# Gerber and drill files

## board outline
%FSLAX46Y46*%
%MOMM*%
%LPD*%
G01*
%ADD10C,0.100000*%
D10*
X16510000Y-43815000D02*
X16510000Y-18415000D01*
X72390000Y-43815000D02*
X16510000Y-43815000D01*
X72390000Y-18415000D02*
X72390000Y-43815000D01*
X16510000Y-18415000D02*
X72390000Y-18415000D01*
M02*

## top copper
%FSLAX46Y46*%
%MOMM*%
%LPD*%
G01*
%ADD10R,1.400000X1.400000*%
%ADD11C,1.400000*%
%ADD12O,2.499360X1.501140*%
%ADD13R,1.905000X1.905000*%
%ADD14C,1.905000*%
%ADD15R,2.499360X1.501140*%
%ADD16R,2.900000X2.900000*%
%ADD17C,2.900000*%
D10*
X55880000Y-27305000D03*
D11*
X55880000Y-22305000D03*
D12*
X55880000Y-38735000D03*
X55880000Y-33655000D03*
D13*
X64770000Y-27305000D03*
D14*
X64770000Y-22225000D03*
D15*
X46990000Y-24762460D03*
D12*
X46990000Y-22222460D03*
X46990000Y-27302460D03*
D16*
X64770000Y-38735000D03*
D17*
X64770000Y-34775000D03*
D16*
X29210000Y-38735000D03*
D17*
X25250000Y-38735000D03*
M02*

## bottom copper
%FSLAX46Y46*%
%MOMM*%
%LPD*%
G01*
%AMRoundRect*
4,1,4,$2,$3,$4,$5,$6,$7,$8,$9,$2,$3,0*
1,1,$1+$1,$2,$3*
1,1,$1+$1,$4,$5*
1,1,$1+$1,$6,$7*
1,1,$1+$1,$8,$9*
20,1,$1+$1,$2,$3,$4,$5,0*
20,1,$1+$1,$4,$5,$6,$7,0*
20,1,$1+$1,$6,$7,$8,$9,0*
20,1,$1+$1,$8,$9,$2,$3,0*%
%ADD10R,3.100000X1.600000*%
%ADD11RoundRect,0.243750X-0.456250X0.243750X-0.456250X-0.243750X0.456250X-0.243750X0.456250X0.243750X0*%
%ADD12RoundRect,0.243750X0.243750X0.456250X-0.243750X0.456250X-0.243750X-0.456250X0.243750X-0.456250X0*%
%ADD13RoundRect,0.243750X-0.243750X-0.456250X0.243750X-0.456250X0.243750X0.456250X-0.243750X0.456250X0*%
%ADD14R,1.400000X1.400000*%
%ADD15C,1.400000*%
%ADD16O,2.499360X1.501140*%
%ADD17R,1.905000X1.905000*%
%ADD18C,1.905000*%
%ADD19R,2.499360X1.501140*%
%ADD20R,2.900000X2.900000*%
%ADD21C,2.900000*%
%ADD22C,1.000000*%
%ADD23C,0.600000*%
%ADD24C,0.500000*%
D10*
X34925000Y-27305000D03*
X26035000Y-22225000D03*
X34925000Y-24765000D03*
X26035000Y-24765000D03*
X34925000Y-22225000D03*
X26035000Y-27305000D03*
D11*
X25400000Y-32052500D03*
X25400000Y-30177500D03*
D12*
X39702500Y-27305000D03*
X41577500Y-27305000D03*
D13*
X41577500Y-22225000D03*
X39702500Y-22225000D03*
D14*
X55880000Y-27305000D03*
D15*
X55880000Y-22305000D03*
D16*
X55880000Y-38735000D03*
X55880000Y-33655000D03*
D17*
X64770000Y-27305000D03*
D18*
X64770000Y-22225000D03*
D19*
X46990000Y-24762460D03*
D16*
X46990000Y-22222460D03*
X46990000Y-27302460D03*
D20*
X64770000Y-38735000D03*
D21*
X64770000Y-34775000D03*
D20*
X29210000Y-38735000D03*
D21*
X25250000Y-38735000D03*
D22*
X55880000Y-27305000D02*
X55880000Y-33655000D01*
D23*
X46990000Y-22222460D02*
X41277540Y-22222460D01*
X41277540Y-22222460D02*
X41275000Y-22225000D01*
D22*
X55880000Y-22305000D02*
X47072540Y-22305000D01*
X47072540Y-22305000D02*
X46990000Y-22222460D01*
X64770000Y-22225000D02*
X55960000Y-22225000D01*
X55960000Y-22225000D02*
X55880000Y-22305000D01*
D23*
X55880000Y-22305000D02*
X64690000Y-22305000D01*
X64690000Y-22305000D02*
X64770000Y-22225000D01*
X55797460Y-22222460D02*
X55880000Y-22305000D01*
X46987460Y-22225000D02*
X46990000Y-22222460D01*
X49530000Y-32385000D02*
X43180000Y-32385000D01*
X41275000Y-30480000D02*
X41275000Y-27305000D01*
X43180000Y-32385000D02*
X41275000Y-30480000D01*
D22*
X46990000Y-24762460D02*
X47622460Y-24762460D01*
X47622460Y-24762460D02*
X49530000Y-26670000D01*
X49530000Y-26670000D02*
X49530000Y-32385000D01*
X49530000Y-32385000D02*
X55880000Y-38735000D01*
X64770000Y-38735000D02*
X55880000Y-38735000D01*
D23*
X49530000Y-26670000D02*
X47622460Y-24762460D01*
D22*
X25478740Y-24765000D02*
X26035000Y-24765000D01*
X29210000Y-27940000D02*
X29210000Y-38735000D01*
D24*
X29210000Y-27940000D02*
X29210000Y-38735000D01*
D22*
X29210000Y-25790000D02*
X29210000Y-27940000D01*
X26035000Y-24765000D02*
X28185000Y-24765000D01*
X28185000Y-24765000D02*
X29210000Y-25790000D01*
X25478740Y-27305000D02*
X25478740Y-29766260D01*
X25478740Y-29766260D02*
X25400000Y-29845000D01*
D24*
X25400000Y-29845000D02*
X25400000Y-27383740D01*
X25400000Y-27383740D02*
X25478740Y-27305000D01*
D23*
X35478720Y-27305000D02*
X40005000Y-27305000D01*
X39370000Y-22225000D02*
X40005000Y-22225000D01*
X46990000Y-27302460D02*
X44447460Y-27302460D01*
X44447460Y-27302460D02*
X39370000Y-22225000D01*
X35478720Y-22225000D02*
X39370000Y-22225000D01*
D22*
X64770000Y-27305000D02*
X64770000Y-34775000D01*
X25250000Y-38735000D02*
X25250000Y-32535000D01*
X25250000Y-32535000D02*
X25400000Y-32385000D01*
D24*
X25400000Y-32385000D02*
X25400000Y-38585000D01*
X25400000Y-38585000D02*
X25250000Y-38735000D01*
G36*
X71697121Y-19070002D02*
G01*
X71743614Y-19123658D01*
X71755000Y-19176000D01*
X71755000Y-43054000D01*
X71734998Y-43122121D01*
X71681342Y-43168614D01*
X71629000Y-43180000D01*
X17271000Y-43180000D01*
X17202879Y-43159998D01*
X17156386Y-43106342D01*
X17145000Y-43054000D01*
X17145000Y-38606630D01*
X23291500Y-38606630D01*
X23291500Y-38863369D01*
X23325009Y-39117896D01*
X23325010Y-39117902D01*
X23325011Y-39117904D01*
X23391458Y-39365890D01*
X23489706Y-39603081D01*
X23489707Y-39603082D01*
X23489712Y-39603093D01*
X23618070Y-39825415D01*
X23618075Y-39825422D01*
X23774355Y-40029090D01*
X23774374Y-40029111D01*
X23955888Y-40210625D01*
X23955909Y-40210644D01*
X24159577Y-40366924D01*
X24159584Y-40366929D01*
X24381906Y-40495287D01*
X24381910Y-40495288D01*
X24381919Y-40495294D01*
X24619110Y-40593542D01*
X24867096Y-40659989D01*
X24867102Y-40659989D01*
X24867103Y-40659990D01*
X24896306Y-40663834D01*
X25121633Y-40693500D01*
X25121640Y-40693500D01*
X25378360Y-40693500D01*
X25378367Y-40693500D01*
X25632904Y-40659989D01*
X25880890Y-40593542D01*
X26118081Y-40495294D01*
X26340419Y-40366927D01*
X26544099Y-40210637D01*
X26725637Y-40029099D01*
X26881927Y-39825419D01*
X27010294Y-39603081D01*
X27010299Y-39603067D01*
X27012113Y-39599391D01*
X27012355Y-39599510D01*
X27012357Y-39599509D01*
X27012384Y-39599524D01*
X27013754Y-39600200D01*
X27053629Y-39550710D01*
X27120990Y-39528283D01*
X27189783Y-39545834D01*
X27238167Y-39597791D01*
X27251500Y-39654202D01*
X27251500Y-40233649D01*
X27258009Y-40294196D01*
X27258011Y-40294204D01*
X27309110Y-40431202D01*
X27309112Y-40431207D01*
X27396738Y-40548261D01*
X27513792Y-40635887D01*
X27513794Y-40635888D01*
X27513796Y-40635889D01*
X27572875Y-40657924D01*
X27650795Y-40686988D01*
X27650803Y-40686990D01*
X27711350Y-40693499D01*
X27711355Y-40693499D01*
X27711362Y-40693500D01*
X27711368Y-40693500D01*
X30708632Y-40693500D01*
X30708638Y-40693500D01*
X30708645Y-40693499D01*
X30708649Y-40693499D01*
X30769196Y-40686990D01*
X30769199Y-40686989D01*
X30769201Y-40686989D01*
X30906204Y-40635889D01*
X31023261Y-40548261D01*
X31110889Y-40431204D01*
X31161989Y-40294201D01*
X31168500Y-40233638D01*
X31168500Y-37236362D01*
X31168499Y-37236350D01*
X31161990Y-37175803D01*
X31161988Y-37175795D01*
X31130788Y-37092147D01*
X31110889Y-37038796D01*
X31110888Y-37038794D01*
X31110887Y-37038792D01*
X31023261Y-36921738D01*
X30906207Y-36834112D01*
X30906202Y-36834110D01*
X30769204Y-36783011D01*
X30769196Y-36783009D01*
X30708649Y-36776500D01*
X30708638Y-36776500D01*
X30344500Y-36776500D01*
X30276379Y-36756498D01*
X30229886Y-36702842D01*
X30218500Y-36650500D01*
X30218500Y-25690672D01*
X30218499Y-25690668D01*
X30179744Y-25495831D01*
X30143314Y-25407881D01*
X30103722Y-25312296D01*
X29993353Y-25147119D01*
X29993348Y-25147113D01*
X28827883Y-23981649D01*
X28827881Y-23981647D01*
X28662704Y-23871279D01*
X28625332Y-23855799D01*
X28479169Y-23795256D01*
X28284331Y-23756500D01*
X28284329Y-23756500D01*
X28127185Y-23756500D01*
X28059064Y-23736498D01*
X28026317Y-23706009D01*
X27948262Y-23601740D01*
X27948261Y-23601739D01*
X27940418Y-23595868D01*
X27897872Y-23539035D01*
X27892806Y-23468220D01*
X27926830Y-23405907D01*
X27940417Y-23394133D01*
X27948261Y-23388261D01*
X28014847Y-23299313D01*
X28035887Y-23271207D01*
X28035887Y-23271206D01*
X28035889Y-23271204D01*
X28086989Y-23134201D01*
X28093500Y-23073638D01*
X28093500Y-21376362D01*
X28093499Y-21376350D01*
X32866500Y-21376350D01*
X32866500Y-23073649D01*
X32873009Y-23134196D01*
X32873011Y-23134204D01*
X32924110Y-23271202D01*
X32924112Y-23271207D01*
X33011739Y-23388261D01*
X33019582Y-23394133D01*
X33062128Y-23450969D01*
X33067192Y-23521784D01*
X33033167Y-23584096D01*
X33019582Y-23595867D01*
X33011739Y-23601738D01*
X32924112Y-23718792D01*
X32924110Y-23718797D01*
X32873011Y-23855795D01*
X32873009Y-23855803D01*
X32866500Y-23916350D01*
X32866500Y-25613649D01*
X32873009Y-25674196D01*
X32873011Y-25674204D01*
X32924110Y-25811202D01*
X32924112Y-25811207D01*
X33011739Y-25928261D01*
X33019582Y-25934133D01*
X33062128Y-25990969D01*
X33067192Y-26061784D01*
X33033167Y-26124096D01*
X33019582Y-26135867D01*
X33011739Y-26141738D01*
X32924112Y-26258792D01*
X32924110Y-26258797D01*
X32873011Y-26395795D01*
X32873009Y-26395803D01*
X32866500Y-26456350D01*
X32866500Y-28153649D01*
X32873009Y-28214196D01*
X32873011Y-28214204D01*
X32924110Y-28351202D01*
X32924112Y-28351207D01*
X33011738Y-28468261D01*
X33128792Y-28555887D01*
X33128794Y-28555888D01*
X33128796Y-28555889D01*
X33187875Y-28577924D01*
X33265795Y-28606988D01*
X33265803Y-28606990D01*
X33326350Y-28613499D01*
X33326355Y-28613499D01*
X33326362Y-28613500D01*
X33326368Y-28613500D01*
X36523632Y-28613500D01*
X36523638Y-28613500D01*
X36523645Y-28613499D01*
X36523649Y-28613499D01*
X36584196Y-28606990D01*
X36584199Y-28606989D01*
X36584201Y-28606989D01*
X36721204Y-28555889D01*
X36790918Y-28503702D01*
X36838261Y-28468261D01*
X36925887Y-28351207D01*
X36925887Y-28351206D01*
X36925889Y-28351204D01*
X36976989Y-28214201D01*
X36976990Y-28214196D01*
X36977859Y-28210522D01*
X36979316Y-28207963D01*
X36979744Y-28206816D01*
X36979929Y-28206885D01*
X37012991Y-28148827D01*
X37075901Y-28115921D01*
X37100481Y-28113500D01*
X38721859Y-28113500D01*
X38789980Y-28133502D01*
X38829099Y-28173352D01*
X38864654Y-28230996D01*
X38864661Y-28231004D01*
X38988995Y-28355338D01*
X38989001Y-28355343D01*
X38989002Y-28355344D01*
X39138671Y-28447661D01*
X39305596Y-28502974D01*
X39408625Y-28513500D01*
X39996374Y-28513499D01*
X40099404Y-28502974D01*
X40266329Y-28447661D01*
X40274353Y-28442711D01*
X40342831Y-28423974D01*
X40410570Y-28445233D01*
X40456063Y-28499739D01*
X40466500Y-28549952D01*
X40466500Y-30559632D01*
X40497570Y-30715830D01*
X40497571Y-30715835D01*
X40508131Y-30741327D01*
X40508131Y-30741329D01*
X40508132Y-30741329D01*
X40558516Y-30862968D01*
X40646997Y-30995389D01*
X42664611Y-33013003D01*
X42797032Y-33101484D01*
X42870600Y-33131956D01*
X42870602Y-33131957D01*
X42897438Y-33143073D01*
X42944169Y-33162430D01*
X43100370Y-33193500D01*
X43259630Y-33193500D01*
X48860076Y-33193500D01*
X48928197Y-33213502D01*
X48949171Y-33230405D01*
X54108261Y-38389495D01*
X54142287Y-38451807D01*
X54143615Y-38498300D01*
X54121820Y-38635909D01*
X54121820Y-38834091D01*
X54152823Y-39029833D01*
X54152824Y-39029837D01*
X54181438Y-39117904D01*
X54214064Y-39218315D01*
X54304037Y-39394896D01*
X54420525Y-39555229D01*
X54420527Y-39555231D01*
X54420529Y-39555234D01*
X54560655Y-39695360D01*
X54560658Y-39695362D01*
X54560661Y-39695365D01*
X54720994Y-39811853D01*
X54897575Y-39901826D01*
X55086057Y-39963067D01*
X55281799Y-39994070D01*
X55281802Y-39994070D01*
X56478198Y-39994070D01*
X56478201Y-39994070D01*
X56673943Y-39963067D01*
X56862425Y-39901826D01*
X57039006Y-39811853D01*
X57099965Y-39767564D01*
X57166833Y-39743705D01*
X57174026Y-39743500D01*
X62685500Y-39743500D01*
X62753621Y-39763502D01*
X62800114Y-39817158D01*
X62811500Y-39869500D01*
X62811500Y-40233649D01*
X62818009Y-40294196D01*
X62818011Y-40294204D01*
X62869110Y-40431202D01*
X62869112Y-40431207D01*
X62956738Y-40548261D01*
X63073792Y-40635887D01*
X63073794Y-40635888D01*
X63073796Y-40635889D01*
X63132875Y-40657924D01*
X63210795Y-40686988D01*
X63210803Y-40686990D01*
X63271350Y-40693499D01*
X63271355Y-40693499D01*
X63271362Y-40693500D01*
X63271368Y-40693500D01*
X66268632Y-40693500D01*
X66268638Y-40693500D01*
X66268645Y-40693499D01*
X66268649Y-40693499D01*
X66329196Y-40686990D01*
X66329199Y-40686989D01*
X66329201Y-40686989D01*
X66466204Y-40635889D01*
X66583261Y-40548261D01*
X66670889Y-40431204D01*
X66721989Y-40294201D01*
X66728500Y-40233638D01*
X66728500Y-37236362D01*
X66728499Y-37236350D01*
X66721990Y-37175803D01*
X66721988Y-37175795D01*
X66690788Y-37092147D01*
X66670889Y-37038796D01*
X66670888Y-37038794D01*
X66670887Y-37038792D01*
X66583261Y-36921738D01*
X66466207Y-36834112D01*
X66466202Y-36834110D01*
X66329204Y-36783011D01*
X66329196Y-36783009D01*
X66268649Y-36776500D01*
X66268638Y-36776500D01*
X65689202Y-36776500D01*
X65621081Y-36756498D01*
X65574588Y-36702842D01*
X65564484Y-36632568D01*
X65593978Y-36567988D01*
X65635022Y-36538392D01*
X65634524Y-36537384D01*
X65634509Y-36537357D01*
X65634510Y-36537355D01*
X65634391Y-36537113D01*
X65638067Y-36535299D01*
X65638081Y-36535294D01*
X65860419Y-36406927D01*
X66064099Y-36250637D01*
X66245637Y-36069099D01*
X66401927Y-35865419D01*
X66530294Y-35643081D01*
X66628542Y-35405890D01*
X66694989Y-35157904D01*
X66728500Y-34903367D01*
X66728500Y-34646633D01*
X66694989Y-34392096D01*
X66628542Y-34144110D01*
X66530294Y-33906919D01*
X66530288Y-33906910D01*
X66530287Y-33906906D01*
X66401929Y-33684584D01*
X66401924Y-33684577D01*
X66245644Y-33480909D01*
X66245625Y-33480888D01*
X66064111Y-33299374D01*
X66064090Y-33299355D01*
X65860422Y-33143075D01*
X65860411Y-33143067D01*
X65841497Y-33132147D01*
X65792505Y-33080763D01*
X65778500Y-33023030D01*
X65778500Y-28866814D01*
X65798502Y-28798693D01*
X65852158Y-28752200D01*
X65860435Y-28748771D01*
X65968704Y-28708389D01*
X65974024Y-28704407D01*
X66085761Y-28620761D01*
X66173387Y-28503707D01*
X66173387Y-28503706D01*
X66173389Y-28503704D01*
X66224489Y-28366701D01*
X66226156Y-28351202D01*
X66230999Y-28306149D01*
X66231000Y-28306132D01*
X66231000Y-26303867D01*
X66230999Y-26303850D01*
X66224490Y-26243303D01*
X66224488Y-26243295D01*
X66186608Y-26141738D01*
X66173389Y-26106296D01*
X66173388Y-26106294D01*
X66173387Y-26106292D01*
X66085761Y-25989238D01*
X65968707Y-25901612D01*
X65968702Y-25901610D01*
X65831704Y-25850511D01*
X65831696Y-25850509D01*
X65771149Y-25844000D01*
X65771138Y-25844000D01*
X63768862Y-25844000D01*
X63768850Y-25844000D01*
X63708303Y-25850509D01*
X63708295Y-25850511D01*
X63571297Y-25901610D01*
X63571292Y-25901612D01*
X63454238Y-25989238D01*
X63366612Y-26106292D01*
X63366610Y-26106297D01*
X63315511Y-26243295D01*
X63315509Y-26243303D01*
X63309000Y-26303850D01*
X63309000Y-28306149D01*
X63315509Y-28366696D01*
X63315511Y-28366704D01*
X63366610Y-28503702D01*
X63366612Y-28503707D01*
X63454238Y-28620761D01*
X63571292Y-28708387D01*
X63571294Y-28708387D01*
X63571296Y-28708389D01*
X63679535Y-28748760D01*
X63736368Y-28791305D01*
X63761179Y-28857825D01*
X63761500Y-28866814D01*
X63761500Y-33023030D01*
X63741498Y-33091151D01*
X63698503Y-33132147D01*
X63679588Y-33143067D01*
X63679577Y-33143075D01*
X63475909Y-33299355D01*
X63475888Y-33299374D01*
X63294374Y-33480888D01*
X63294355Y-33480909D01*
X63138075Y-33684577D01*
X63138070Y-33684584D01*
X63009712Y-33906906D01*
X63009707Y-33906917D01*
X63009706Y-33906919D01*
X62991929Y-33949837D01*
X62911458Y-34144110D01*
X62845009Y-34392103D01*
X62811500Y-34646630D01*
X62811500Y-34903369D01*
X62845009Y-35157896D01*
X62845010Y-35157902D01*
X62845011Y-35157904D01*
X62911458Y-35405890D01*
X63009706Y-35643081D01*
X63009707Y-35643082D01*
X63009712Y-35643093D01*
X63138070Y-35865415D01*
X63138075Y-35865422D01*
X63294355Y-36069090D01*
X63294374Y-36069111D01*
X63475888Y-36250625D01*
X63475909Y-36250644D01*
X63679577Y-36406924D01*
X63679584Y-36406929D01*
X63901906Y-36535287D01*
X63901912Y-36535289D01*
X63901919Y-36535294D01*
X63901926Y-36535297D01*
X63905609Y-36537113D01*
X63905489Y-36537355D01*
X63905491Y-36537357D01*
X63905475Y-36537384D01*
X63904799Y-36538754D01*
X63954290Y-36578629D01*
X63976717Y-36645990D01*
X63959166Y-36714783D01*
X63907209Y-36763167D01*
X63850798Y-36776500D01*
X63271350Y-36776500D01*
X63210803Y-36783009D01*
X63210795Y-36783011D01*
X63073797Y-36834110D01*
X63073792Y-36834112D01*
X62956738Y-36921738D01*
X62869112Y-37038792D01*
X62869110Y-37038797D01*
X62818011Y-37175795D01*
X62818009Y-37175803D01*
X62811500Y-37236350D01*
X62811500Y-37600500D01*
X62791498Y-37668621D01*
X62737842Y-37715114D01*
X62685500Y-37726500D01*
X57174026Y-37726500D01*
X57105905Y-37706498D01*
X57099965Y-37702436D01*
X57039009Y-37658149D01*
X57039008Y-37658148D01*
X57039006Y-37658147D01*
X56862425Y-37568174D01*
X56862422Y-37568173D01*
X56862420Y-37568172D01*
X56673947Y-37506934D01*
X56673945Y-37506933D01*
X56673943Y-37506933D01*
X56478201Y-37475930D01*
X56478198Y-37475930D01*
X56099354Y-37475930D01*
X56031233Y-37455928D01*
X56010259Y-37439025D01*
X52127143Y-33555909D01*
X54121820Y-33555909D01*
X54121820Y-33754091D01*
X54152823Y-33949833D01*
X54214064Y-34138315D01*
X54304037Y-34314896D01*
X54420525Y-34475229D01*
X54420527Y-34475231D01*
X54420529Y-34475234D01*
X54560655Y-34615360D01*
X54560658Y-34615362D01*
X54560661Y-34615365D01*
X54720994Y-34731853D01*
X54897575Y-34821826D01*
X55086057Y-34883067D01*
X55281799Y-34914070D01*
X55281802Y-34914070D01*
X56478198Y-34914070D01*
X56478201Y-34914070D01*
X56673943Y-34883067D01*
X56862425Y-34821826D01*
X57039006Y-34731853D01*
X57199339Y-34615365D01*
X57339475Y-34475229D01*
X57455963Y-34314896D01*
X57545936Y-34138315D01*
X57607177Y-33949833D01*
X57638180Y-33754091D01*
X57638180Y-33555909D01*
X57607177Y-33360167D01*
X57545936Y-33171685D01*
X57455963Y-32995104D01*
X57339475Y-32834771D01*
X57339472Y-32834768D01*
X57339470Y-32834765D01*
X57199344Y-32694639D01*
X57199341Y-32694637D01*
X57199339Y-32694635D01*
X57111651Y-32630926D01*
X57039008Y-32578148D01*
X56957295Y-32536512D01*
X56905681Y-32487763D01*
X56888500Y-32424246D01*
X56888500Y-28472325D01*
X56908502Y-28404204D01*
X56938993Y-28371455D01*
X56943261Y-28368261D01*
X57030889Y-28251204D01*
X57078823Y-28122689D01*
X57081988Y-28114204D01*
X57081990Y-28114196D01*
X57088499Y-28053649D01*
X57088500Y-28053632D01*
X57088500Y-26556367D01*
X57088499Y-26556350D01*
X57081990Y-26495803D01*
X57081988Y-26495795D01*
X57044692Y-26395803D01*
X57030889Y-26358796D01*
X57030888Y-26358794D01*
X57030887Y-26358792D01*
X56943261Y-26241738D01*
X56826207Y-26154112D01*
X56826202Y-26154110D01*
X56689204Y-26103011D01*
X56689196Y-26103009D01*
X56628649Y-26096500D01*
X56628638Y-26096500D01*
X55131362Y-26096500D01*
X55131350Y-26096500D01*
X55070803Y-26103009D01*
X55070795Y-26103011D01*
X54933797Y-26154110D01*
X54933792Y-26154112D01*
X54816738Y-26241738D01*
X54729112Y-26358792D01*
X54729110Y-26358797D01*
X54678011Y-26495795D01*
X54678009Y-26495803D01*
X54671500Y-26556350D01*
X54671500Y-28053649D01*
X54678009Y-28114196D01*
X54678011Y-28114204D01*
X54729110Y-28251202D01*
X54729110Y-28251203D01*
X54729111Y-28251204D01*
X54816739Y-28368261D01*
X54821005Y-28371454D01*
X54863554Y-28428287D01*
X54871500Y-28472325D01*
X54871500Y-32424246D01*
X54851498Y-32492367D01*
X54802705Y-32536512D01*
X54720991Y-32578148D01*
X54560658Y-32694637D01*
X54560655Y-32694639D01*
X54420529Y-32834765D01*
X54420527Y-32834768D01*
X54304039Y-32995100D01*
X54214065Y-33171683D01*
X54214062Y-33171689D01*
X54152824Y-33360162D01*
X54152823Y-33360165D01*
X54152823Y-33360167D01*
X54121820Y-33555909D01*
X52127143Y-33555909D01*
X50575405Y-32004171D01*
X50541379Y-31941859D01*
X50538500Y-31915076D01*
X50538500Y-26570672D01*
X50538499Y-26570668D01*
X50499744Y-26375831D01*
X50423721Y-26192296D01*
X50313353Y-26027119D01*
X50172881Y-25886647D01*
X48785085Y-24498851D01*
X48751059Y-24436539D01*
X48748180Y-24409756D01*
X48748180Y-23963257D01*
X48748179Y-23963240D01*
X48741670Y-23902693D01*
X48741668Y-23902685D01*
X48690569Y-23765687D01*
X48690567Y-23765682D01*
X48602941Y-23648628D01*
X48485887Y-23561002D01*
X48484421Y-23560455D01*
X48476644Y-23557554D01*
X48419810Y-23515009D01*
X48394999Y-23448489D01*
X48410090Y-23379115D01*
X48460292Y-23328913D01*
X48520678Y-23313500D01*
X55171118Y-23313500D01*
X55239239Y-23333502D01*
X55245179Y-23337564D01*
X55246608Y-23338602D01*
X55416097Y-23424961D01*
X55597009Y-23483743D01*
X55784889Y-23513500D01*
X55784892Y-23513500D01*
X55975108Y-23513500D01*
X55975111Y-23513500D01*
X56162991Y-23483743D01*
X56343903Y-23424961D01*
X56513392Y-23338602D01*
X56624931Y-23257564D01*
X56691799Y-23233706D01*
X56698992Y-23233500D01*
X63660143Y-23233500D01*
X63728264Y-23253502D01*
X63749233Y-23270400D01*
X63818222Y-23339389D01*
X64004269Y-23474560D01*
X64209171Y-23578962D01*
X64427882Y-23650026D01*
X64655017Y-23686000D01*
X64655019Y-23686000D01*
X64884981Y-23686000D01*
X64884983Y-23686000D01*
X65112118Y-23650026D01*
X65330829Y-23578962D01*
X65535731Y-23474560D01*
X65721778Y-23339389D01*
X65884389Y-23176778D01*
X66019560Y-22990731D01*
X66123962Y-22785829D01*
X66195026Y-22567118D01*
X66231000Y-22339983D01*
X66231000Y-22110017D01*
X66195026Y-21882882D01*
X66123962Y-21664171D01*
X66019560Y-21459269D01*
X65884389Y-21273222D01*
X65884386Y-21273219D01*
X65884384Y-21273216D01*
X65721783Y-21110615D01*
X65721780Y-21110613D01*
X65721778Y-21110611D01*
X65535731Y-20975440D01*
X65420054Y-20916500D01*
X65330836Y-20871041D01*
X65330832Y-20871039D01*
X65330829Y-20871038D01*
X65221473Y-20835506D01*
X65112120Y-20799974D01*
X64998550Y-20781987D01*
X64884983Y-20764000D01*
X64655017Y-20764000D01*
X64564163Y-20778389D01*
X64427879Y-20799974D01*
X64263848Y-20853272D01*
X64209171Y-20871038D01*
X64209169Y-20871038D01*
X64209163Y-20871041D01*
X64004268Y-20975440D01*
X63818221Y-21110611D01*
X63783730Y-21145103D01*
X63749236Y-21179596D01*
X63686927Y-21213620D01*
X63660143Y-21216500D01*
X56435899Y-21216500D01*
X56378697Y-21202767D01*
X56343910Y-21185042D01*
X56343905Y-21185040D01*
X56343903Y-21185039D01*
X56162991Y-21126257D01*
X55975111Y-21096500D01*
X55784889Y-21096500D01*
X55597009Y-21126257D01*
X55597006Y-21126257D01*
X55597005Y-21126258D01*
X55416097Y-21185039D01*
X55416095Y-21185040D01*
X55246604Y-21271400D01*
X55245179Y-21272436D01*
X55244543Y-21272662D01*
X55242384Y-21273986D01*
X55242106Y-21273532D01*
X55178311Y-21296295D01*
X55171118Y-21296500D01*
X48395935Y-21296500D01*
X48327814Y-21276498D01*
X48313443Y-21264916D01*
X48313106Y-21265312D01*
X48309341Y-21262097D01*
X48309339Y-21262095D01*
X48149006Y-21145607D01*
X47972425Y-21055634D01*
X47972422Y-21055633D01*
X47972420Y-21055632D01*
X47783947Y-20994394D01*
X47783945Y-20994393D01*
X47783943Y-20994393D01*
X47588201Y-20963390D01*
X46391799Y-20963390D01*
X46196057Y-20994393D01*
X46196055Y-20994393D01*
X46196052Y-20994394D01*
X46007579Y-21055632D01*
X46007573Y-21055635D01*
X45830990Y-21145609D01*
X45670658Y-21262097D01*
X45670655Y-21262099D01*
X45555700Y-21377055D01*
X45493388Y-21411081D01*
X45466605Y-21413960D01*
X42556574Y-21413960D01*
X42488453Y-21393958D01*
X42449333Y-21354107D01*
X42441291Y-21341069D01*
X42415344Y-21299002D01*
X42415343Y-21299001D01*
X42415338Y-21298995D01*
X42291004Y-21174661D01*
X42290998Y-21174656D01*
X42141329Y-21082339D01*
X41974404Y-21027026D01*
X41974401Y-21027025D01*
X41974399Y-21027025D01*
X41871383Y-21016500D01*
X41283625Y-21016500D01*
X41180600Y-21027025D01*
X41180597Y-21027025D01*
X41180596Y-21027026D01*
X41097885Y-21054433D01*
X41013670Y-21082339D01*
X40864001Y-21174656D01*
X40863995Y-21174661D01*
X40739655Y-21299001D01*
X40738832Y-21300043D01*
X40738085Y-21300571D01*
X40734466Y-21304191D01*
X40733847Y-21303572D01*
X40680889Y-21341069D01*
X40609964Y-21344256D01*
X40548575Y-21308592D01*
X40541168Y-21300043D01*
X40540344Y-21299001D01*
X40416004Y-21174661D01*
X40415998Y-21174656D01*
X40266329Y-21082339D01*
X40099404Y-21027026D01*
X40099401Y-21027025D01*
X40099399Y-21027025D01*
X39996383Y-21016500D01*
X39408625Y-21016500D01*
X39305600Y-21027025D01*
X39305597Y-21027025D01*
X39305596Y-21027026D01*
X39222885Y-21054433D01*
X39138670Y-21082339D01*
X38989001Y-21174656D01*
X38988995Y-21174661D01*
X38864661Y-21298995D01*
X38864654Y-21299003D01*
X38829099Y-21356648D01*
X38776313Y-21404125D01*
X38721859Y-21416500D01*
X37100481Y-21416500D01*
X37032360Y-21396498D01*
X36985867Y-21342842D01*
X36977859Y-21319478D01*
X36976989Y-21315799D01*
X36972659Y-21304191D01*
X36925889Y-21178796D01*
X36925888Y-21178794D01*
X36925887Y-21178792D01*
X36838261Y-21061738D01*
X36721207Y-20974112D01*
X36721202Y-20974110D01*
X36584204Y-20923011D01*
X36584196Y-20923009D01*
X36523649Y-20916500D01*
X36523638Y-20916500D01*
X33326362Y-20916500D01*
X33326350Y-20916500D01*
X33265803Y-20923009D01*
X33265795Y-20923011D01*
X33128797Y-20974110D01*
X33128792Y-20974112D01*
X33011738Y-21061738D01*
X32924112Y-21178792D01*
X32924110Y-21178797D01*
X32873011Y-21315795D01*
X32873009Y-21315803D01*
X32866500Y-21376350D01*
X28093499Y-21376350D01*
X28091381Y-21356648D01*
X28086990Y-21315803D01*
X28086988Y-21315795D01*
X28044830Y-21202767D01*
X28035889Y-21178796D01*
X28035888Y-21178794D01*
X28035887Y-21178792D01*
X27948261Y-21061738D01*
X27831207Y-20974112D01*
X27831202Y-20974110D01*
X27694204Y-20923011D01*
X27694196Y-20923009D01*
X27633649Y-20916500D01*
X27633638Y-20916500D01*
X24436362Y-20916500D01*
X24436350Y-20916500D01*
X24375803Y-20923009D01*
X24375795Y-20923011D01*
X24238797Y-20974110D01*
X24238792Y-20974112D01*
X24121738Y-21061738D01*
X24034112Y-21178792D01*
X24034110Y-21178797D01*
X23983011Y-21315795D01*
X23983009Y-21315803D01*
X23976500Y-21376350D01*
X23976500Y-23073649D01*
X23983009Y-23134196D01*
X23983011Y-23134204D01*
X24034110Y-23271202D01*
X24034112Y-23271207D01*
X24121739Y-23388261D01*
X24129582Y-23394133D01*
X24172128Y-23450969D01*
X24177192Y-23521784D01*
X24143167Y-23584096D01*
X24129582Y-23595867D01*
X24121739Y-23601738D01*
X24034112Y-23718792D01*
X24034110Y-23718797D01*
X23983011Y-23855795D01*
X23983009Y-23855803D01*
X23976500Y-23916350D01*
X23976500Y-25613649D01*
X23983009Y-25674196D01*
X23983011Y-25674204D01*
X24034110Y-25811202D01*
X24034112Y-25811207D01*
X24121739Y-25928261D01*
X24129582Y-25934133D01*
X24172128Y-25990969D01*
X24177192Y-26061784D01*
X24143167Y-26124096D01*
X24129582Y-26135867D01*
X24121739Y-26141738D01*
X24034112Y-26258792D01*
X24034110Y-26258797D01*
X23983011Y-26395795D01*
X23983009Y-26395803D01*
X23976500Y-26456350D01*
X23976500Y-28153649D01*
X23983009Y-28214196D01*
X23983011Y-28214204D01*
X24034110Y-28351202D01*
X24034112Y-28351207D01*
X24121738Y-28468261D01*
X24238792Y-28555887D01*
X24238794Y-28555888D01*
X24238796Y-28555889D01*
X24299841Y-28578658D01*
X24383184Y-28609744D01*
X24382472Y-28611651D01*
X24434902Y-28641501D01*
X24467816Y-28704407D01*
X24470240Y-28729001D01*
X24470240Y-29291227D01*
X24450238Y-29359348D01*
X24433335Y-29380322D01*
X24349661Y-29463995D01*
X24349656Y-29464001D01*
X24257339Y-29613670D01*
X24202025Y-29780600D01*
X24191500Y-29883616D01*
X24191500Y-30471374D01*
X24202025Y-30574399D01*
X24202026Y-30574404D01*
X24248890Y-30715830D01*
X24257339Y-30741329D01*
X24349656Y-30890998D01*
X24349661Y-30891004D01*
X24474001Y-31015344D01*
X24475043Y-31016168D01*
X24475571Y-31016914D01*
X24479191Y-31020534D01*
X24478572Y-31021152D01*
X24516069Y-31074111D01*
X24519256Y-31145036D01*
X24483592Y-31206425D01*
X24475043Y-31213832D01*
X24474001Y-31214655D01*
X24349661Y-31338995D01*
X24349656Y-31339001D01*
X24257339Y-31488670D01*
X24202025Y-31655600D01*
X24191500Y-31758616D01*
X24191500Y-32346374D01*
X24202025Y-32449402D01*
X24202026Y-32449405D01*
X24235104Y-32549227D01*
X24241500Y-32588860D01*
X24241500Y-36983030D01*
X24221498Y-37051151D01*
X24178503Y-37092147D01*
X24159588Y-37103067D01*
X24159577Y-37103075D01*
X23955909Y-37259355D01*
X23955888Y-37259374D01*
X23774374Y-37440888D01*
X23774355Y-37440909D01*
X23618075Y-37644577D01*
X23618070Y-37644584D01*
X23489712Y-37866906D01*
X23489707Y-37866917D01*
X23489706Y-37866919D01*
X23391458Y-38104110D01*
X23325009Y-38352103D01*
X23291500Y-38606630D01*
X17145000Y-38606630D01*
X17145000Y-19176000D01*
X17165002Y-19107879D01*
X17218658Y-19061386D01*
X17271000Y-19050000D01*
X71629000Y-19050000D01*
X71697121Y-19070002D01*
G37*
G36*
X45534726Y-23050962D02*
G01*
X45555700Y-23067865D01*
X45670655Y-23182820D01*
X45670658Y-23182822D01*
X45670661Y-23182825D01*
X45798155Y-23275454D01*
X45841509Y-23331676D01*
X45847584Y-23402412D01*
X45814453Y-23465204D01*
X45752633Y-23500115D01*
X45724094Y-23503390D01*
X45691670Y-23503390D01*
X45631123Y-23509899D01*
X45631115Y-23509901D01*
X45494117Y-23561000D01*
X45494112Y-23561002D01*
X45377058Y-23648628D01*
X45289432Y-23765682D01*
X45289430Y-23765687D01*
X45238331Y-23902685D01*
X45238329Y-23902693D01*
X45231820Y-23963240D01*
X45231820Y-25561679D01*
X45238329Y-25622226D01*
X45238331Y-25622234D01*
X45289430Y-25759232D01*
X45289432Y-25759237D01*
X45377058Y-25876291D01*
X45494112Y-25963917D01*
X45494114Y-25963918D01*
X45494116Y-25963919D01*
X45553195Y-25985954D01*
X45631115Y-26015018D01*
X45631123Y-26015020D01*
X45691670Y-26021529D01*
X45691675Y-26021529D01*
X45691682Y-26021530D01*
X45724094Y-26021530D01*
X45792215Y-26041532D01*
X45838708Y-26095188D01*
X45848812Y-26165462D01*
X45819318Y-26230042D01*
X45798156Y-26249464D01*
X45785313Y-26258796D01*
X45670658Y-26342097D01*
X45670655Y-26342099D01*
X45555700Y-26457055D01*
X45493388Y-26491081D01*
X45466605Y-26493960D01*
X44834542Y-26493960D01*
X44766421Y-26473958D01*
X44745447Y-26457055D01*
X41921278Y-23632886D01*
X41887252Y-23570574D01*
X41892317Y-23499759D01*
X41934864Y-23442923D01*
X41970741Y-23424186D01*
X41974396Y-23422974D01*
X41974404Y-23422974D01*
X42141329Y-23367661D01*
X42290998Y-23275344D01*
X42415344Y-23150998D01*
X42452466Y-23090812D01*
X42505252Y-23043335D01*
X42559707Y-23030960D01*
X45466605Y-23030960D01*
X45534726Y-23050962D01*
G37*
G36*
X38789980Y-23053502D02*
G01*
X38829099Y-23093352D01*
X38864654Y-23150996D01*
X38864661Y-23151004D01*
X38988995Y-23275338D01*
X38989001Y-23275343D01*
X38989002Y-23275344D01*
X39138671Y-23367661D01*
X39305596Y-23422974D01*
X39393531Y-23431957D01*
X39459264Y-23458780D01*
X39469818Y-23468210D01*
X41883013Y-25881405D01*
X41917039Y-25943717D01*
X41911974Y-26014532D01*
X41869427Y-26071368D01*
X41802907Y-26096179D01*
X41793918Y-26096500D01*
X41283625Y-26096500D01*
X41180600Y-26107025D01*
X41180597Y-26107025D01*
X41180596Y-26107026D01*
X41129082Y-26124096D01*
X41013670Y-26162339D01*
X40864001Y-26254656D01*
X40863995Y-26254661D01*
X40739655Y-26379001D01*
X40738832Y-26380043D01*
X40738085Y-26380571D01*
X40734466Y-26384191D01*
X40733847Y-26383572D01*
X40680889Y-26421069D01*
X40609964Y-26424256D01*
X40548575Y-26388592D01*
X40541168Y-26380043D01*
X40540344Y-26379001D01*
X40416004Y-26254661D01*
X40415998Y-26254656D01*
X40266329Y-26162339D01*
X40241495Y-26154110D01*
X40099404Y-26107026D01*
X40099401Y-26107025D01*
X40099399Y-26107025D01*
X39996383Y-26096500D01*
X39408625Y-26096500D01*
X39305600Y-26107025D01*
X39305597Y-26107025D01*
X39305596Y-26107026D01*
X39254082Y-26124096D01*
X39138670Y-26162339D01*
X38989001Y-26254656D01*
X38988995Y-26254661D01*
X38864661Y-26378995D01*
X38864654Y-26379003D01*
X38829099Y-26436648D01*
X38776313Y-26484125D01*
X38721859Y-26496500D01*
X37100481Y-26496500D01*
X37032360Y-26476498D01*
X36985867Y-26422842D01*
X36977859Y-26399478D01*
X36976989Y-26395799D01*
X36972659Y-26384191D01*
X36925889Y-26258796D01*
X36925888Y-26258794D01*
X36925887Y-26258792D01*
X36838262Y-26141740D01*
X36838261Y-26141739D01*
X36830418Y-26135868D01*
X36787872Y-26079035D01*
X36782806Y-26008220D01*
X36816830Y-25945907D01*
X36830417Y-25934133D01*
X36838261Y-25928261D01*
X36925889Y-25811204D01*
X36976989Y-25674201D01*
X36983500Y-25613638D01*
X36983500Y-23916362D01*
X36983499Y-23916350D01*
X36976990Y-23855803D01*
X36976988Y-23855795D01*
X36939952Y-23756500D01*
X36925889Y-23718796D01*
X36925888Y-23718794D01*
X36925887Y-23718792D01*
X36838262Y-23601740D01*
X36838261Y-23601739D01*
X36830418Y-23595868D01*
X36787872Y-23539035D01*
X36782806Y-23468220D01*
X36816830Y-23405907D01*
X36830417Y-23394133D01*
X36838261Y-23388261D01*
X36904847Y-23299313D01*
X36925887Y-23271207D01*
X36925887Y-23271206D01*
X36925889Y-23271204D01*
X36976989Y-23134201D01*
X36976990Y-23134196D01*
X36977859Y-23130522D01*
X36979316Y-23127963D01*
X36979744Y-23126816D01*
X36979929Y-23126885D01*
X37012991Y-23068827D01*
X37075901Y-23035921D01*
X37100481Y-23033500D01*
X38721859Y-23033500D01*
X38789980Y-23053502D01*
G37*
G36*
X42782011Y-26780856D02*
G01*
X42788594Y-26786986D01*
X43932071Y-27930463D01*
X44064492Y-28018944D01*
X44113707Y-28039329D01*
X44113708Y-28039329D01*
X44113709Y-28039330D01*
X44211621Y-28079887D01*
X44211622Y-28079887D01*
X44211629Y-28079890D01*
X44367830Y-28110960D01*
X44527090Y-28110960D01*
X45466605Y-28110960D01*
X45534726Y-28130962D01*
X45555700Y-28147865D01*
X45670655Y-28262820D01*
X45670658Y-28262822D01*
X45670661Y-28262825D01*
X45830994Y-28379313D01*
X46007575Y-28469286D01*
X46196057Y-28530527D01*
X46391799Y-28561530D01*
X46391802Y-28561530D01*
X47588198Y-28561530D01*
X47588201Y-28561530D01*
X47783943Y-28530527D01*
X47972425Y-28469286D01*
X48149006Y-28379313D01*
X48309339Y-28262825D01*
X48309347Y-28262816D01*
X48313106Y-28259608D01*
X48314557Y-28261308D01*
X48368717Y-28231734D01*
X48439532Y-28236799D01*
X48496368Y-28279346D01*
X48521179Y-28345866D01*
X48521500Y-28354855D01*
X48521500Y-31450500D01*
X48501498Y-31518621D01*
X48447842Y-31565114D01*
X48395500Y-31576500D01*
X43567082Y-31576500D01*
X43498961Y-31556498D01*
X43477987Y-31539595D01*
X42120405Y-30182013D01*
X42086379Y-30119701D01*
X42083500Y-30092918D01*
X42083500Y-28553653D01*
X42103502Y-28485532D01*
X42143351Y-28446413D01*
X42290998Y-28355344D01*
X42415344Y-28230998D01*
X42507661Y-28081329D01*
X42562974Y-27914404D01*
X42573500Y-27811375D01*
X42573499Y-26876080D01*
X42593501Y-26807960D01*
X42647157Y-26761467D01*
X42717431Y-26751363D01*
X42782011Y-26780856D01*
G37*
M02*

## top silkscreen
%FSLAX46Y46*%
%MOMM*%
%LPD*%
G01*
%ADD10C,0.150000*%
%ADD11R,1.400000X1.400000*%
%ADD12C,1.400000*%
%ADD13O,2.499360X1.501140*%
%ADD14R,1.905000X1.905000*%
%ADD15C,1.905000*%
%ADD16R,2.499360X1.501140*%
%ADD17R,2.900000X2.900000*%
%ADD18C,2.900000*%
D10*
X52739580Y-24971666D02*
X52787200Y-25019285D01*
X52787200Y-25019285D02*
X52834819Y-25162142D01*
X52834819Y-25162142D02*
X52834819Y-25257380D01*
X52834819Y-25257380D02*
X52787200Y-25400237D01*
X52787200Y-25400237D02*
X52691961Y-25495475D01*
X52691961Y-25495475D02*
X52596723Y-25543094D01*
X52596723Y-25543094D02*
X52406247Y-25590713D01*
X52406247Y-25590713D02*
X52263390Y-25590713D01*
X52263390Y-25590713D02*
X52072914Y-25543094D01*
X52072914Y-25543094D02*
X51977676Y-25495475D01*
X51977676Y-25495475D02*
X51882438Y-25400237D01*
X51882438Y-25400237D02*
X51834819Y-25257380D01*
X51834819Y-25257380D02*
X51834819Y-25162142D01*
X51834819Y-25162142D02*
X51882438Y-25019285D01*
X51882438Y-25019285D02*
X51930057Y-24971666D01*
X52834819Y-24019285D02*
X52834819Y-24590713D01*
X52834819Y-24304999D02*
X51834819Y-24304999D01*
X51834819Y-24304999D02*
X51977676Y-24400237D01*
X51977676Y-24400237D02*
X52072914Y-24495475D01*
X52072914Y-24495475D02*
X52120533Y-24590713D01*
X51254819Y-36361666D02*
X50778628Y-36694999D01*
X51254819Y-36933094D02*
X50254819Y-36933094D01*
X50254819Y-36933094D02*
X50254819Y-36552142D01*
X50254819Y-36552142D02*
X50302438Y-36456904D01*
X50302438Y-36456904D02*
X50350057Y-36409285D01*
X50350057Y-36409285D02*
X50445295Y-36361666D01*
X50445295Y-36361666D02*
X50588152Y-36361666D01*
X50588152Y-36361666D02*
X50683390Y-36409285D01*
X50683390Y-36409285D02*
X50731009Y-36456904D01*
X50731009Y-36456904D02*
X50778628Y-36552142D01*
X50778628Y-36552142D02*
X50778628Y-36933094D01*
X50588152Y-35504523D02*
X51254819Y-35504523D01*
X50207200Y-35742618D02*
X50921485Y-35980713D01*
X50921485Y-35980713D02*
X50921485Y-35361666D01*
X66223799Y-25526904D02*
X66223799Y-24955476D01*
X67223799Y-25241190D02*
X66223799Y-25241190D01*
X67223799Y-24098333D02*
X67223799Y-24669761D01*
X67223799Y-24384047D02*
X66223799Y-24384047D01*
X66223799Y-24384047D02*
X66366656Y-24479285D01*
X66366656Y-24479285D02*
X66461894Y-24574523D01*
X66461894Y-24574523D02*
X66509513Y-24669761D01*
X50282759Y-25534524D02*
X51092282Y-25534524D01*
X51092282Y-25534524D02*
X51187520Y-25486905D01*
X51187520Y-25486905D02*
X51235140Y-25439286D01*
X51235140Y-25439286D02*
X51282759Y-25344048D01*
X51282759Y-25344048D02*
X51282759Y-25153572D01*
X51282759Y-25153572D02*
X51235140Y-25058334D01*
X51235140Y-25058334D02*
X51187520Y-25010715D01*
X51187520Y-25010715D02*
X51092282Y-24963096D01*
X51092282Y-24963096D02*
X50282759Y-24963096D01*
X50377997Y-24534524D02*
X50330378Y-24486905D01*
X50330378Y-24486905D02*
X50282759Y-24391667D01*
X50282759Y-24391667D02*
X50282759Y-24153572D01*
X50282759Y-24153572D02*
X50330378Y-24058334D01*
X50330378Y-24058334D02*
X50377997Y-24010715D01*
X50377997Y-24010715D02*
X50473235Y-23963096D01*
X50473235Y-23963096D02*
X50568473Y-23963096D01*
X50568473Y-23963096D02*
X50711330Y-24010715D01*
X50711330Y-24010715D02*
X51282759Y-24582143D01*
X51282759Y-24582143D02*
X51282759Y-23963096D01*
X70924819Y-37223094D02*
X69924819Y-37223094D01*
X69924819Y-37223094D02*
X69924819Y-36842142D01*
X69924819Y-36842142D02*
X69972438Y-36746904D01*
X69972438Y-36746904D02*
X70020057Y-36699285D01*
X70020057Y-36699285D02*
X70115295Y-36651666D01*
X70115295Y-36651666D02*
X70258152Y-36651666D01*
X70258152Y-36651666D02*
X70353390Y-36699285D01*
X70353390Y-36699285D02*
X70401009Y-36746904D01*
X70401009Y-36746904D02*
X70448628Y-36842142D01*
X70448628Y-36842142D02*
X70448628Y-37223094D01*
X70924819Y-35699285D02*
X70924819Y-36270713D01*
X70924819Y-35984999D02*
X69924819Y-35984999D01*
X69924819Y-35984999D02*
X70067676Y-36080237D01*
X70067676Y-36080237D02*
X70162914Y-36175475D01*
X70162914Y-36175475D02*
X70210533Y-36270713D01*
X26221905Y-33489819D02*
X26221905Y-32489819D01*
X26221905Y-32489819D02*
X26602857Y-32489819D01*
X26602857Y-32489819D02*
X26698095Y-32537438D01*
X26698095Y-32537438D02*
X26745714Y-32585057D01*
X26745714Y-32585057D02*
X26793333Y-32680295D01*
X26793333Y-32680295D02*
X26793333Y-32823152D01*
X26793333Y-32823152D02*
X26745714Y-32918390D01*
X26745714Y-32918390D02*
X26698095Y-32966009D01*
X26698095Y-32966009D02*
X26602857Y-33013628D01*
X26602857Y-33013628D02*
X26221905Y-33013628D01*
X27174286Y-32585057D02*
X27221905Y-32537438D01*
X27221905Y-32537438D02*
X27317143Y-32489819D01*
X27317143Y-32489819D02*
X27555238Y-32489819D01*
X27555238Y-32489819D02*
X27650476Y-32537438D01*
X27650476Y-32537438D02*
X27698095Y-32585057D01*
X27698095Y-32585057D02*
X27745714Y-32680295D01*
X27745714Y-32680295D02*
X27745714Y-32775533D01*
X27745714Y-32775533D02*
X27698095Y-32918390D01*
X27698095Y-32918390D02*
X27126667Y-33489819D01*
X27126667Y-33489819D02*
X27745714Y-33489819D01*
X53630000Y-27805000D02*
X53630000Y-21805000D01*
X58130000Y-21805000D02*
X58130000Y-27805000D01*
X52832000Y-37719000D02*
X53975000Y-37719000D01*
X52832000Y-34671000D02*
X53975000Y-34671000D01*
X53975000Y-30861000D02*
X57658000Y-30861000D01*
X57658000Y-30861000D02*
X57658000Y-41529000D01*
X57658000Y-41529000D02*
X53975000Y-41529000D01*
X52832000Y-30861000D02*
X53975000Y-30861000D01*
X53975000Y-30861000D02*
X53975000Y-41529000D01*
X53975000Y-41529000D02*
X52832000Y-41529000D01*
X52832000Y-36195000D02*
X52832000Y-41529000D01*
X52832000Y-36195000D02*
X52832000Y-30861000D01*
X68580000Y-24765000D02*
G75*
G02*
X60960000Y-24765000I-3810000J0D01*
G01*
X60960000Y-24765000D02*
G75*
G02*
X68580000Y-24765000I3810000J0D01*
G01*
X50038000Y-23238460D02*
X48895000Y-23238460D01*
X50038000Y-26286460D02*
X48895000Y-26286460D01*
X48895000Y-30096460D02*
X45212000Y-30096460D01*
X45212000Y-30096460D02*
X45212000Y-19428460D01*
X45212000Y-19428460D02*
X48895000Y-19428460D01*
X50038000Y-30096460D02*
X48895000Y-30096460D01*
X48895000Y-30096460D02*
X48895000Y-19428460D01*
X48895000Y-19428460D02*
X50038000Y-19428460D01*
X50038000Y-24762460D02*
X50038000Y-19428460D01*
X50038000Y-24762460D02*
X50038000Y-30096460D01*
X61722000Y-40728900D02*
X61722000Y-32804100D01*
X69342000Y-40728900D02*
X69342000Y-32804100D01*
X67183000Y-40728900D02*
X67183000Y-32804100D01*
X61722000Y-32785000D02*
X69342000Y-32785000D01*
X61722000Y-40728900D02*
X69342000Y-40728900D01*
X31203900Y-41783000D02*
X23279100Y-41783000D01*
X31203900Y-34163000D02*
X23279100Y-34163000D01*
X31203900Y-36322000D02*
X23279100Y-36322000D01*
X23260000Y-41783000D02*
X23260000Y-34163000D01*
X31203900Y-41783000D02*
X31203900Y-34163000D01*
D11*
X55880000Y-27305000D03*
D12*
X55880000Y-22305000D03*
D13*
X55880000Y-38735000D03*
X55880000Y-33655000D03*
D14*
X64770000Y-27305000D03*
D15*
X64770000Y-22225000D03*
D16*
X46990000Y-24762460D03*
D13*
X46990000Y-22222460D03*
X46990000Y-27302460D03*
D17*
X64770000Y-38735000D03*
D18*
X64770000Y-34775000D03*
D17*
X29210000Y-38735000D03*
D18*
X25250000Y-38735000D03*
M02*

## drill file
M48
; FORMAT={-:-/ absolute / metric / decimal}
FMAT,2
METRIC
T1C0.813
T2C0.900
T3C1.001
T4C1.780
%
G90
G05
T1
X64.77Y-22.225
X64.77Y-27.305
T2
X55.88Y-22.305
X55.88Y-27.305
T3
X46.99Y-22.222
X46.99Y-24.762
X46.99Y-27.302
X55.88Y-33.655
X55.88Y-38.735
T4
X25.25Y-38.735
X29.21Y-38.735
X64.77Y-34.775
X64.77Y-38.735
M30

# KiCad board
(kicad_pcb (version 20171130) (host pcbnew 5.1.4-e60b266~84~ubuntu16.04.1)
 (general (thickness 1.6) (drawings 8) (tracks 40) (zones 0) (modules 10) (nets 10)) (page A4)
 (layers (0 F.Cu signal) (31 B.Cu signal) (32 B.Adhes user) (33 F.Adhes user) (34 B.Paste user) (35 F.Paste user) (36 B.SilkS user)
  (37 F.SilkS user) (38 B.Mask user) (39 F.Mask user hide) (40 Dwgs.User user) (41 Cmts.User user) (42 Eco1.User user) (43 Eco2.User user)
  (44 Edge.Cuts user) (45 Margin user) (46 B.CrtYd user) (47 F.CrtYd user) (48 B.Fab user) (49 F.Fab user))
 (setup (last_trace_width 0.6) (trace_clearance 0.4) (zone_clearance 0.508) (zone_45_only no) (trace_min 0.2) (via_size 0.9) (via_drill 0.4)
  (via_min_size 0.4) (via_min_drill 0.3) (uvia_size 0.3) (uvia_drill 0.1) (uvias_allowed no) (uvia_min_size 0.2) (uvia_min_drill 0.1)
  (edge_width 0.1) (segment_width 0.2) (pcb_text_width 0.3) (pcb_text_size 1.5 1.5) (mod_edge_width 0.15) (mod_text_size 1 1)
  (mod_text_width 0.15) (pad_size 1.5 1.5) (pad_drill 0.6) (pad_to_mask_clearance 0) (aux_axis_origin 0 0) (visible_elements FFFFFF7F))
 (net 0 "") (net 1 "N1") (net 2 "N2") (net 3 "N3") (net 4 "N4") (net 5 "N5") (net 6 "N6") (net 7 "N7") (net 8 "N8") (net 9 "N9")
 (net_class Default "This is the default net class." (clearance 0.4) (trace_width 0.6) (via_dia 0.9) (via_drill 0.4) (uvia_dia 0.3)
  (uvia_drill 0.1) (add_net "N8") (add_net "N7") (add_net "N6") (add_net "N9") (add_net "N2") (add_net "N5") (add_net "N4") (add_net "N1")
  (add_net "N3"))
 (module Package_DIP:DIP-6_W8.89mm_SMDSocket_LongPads (layer B.Cu) (at 30.48 24.765)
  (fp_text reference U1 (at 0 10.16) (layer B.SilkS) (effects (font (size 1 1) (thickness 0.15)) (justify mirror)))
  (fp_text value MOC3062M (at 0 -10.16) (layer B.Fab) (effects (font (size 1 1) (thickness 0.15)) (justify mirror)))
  (pad 6 smd rect (at 4.445 2.54) (size 3.1 1.6) (layers B.Cu B.Paste B.Mask) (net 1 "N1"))
  (pad 3 smd rect (at -4.445 -2.54) (size 3.1 1.6) (layers B.Cu B.Paste B.Mask))
  (pad 5 smd rect (at 4.445 0) (size 3.1 1.6) (layers B.Cu B.Paste B.Mask))
  (pad 2 smd rect (at -4.445 0) (size 3.1 1.6) (layers B.Cu B.Paste B.Mask) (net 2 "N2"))
  (pad 4 smd rect (at 4.445 -2.54) (size 3.1 1.6) (layers B.Cu B.Paste B.Mask) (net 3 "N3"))
  (pad 1 smd rect (at -4.445 2.54) (size 3.1 1.6) (layers B.Cu B.Paste B.Mask) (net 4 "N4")))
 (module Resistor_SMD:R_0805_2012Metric (layer B.Cu) (at 25.4 31.115 270)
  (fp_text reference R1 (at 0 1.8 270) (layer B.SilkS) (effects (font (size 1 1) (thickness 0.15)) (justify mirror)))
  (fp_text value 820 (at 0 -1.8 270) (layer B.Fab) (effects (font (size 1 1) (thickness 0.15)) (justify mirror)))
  (pad 2 smd roundrect (at 0.9375 0 270) (size 0.975 1.4) (layers B.Cu B.Paste B.Mask) (roundrect_rratio 0.25) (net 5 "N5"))
  (pad 1 smd roundrect (at -0.9375 0 270) (size 0.975 1.4) (layers B.Cu B.Paste B.Mask) (roundrect_rratio 0.25) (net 4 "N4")))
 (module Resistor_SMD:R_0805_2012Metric (layer B.Cu) (at 40.64 27.305 180)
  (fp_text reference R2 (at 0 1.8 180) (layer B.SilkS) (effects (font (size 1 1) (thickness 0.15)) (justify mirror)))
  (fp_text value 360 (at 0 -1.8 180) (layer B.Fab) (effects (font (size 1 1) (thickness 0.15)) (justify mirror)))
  (pad 2 smd roundrect (at 0.9375 0 180) (size 0.975 1.4) (layers B.Cu B.Paste B.Mask) (roundrect_rratio 0.25) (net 1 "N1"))
  (pad 1 smd roundrect (at -0.9375 0 180) (size 0.975 1.4) (layers B.Cu B.Paste B.Mask) (roundrect_rratio 0.25) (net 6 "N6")))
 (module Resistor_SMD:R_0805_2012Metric (layer B.Cu) (at 40.64 22.225)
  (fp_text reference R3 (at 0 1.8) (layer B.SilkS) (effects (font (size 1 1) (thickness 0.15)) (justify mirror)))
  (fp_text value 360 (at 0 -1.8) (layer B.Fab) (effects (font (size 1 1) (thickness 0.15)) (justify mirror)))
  (pad 2 smd roundrect (at 0.9375 0) (size 0.975 1.4) (layers B.Cu B.Paste B.Mask) (roundrect_rratio 0.25) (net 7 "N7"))
  (pad 1 smd roundrect (at -0.9375 0) (size 0.975 1.4) (layers B.Cu B.Paste B.Mask) (roundrect_rratio 0.25) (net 3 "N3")))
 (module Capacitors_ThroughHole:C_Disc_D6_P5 (layer F.Cu) (at 55.88 27.305 90)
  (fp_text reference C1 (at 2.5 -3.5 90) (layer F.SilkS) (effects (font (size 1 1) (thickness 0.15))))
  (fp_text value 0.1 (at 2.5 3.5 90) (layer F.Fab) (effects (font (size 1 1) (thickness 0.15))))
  (fp_line (start -0.5 -2.25) (end 5.5 -2.25) (layer F.SilkS) (width 0.15))
  (fp_line (start 5.5 2.25) (end -0.5 2.25) (layer F.SilkS) (width 0.15))
  (pad 1 thru_hole rect (at 0 0 90) (size 1.4 1.4) (drill 0.9) (layers *.Cu *.Mask F.SilkS) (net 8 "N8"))
  (pad 2 thru_hole circle (at 5 0 90) (size 1.4 1.4) (drill 0.9) (layers *.Cu *.Mask F.SilkS) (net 7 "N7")))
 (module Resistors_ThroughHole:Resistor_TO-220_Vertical (layer F.Cu) (at 55.88 36.195 90)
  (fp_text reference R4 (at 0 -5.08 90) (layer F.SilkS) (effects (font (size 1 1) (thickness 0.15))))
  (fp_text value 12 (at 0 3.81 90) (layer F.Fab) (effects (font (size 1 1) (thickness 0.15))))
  (fp_line (start -1.524 -3.048) (end -1.524 -1.905) (layer F.SilkS) (width 0.15))
  (fp_line (start 1.524 -3.048) (end 1.524 -1.905) (layer F.SilkS) (width 0.15))
  (fp_line (start 5.334 -1.905) (end 5.334 1.778) (layer F.SilkS) (width 0.15))
  (fp_line (start 5.334 1.778) (end -5.334 1.778) (layer F.SilkS) (width 0.15))
  (fp_line (start -5.334 1.778) (end -5.334 -1.905) (layer F.SilkS) (width 0.15))
  (fp_line (start 5.334 -3.048) (end 5.334 -1.905) (layer F.SilkS) (width 0.15))
  (fp_line (start 5.334 -1.905) (end -5.334 -1.905) (layer F.SilkS) (width 0.15))
  (fp_line (start -5.334 -1.905) (end -5.334 -3.048) (layer F.SilkS) (width 0.15))
  (fp_line (start 0 -3.048) (end -5.334 -3.048) (layer F.SilkS) (width 0.15))
  (fp_line (start 0 -3.048) (end 5.334 -3.048) (layer F.SilkS) (width 0.15))
  (pad 1 thru_hole oval (at -2.54 0 180) (size 2.49936 1.50114) (drill 1.00076) (layers *.Cu *.Mask F.SilkS) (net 6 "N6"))
  (pad 2 thru_hole oval (at 2.54 0 180) (size 2.49936 1.50114) (drill 1.00076) (layers *.Cu *.Mask F.SilkS) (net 8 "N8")))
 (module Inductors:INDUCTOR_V (layer F.Cu) (at 64.77 24.765 90)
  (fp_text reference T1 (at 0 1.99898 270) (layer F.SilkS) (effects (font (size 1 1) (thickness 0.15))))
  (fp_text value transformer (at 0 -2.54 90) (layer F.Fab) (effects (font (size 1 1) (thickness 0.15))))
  (fp_circle (center 0 0) (end 3.81 0) (layer F.SilkS) (width 0.15))
  (pad 1 thru_hole rect (at -2.54 0 90) (size 1.905 1.905) (drill 0.8128) (layers *.Cu *.Mask F.SilkS) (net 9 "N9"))
  (pad 2 thru_hole circle (at 2.54 0 90) (size 1.905 1.905) (drill 0.8128) (layers *.Cu *.Mask F.SilkS) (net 7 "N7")))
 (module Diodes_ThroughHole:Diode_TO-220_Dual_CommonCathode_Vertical (layer F.Cu) (at 46.99 22.225 270)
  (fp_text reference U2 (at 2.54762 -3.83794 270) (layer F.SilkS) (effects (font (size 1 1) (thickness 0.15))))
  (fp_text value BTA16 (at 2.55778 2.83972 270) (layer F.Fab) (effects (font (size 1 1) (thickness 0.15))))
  (fp_line (start 1.01346 -3.048) (end 1.01346 -1.905) (layer F.SilkS) (width 0.15))
  (fp_line (start 4.06146 -3.048) (end 4.06146 -1.905) (layer F.SilkS) (width 0.15))
  (fp_line (start 7.87146 -1.905) (end 7.87146 1.778) (layer F.SilkS) (width 0.15))
  (fp_line (start 7.87146 1.778) (end -2.79654 1.778) (layer F.SilkS) (width 0.15))
  (fp_line (start -2.79654 1.778) (end -2.79654 -1.905) (layer F.SilkS) (width 0.15))
  (fp_line (start 7.87146 -3.048) (end 7.87146 -1.905) (layer F.SilkS) (width 0.15))
  (fp_line (start 7.87146 -1.905) (end -2.79654 -1.905) (layer F.SilkS) (width 0.15))
  (fp_line (start -2.79654 -1.905) (end -2.79654 -3.048) (layer F.SilkS) (width 0.15))
  (fp_line (start 2.53746 -3.048) (end -2.79654 -3.048) (layer F.SilkS) (width 0.15))
  (fp_line (start 2.53746 -3.048) (end 7.87146 -3.048) (layer F.SilkS) (width 0.15))
  (pad 2 thru_hole rect (at 2.53746 0) (size 2.49936 1.50114) (drill 1.00076) (layers *.Cu *.Mask F.SilkS) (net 6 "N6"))
  (pad 1 thru_hole oval (at -0.00254 0) (size 2.49936 1.50114) (drill 1.00076) (layers *.Cu *.Mask F.SilkS) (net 7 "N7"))
  (pad 3 thru_hole oval (at 5.07746 0) (size 2.49936 1.50114) (drill 1.00076) (layers *.Cu *.Mask F.SilkS) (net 3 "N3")))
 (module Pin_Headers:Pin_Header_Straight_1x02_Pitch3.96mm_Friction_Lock (layer F.Cu) (at 64.77 38.735 90)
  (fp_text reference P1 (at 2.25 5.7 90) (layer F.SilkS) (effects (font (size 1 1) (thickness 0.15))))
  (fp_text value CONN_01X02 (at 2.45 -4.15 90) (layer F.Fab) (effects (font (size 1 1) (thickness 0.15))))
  (fp_line (start -1.9939 -3.048) (end 5.9309 -3.048) (layer F.SilkS) (width 0.15))
  (fp_line (start -1.9939 4.572) (end 5.9309 4.572) (layer F.SilkS) (width 0.15))
  (fp_line (start -1.9939 2.413) (end 5.9309 2.413) (layer F.SilkS) (width 0.15))
  (fp_line (start 5.95 -3.048) (end 5.95 4.572) (layer F.SilkS) (width 0.15))
  (fp_line (start -1.9939 -3.048) (end -1.9939 4.572) (layer F.SilkS) (width 0.15))
  (pad 1 thru_hole rect (at 0 0 90) (size 2.9 2.9) (drill 1.78) (layers *.Cu *.Mask F.SilkS) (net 6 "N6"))
  (pad 2 thru_hole circle (at 3.96 0 90) (size 2.9 2.9) (drill 1.78) (layers *.Cu *.Mask F.SilkS) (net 9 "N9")))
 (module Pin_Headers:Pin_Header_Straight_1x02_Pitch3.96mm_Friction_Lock (layer F.Cu) (at 29.21 38.735 180)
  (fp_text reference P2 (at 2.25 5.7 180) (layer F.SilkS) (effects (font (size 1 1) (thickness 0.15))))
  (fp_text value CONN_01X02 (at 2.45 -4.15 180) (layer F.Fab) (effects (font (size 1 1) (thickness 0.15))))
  (fp_line (start -1.9939 -3.048) (end 5.9309 -3.048) (layer F.SilkS) (width 0.15))
  (fp_line (start -1.9939 4.572) (end 5.9309 4.572) (layer F.SilkS) (width 0.15))
  (fp_line (start -1.9939 2.413) (end 5.9309 2.413) (layer F.SilkS) (width 0.15))
  (fp_line (start 5.95 -3.048) (end 5.95 4.572) (layer F.SilkS) (width 0.15))
  (fp_line (start -1.9939 -3.048) (end -1.9939 4.572) (layer F.SilkS) (width 0.15))
  (pad 1 thru_hole rect (at 0 0 180) (size 2.9 2.9) (drill 1.78) (layers *.Cu *.Mask F.SilkS) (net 2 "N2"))
  (pad 2 thru_hole circle (at 3.96 0 180) (size 2.9 2.9) (drill 1.78) (layers *.Cu *.Mask F.SilkS) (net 5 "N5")))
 (gr_line (start 16.51 43.815) (end 16.51 18.415) (layer Edge.Cuts) (width 0.1))
 (gr_line (start 72.39 43.815) (end 16.51 43.815) (layer Edge.Cuts) (width 0.1))
 (gr_line (start 72.39 18.415) (end 72.39 43.815) (layer Edge.Cuts) (width 0.1))
 (gr_line (start 16.51 18.415) (end 72.39 18.415) (layer Edge.Cuts) (width 0.1))
 (segment (start 55.88 27.305) (end 55.88 33.655) (width 1) (layer B.Cu) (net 8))
 (segment (start 46.99 22.22246) (end 41.27754 22.22246) (width 0.6) (layer B.Cu) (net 7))
 (segment (start 41.27754 22.22246) (end 41.275 22.225) (width 0.6) (layer B.Cu) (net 7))
 (segment (start 55.88 22.305) (end 47.07254 22.305) (width 1) (layer B.Cu) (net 7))
 (segment (start 47.07254 22.305) (end 46.99 22.22246) (width 1) (layer B.Cu) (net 7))
 (segment (start 64.77 22.225) (end 55.96 22.225) (width 1) (layer B.Cu) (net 7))
 (segment (start 55.96 22.225) (end 55.88 22.305) (width 1) (layer B.Cu) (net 7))
 (segment (start 55.88 22.305) (end 64.69 22.305) (width 0.6) (layer B.Cu) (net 7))
 (segment (start 64.69 22.305) (end 64.77 22.225) (width 0.6) (layer B.Cu) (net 7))
 (segment (start 55.79746 22.22246) (end 55.88 22.305) (width 0.6) (layer B.Cu) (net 7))
 (segment (start 46.98746 22.225) (end 46.99 22.22246) (width 0.6) (layer B.Cu) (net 7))
 (segment (start 49.53 32.385) (end 43.18 32.385) (width 0.6) (layer B.Cu) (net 6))
 (segment (start 41.275 30.48) (end 41.275 27.305) (width 0.6) (layer B.Cu) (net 6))
 (segment (start 43.18 32.385) (end 41.275 30.48) (width 0.6) (layer B.Cu) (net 6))
 (segment (start 46.99 24.76246) (end 47.62246 24.76246) (width 1) (layer B.Cu) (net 6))
 (segment (start 47.62246 24.76246) (end 49.53 26.67) (width 1) (layer B.Cu) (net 6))
 (segment (start 49.53 26.67) (end 49.53 32.385) (width 1) (layer B.Cu) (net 6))
 (segment (start 49.53 32.385) (end 55.88 38.735) (width 1) (layer B.Cu) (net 6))
 (segment (start 64.77 38.735) (end 55.88 38.735) (width 1) (layer B.Cu) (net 6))
 (segment (start 49.53 26.67) (end 47.62246 24.76246) (width 0.6) (layer B.Cu) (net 6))
 (segment (start 25.47874 24.765) (end 26.035 24.765) (width 1) (layer B.Cu) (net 2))
 (segment (start 29.21 27.94) (end 29.21 38.735) (width 1) (layer B.Cu) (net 2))
 (segment (start 29.21 27.94) (end 29.21 38.735) (width 0.5) (layer B.Cu) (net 2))
 (segment (start 29.21 25.79) (end 29.21 27.94) (width 1) (layer B.Cu) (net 2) (status 1000000))
 (segment (start 26.035 24.765) (end 28.185 24.765) (width 1) (layer B.Cu) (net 2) (status 1000000))
 (segment (start 28.185 24.765) (end 29.21 25.79) (width 1) (layer B.Cu) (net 2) (status 1000000))
 (segment (start 25.47874 27.305) (end 25.47874 29.76626) (width 1) (layer B.Cu) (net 4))
 (segment (start 25.47874 29.76626) (end 25.4 29.845) (width 1) (layer B.Cu) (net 4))
 (segment (start 25.4 29.845) (end 25.4 27.38374) (width 0.5) (layer B.Cu) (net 4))
 (segment (start 25.4 27.38374) (end 25.47874 27.305) (width 0.5) (layer B.Cu) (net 4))
 (segment (start 35.47872 27.305) (end 40.005 27.305) (width 0.6) (layer B.Cu) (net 1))
 (segment (start 39.37 22.225) (end 40.005 22.225) (width 0.6) (layer B.Cu) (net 3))
 (segment (start 46.99 27.30246) (end 44.44746 27.30246) (width 0.6) (layer B.Cu) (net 3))
 (segment (start 44.44746 27.30246) (end 39.37 22.225) (width 0.6) (layer B.Cu) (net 3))
 (segment (start 35.47872 22.225) (end 39.37 22.225) (width 0.6) (layer B.Cu) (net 3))
 (segment (start 64.77 27.305) (end 64.77 34.775) (width 1) (layer B.Cu) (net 9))
 (segment (start 25.25 38.735) (end 25.25 32.535) (width 1) (layer B.Cu) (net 5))
 (segment (start 25.25 32.535) (end 25.4 32.385) (width 1) (layer B.Cu) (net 5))
 (segment (start 25.4 32.385) (end 25.4 38.585) (width 0.5) (layer B.Cu) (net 5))
 (segment (start 25.4 38.585) (end 25.25 38.735) (width 0.5) (layer B.Cu) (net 5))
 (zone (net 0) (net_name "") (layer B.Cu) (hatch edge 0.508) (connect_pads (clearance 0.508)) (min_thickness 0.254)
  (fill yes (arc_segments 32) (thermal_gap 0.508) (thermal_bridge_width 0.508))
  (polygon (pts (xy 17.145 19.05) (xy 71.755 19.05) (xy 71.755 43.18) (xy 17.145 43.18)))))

